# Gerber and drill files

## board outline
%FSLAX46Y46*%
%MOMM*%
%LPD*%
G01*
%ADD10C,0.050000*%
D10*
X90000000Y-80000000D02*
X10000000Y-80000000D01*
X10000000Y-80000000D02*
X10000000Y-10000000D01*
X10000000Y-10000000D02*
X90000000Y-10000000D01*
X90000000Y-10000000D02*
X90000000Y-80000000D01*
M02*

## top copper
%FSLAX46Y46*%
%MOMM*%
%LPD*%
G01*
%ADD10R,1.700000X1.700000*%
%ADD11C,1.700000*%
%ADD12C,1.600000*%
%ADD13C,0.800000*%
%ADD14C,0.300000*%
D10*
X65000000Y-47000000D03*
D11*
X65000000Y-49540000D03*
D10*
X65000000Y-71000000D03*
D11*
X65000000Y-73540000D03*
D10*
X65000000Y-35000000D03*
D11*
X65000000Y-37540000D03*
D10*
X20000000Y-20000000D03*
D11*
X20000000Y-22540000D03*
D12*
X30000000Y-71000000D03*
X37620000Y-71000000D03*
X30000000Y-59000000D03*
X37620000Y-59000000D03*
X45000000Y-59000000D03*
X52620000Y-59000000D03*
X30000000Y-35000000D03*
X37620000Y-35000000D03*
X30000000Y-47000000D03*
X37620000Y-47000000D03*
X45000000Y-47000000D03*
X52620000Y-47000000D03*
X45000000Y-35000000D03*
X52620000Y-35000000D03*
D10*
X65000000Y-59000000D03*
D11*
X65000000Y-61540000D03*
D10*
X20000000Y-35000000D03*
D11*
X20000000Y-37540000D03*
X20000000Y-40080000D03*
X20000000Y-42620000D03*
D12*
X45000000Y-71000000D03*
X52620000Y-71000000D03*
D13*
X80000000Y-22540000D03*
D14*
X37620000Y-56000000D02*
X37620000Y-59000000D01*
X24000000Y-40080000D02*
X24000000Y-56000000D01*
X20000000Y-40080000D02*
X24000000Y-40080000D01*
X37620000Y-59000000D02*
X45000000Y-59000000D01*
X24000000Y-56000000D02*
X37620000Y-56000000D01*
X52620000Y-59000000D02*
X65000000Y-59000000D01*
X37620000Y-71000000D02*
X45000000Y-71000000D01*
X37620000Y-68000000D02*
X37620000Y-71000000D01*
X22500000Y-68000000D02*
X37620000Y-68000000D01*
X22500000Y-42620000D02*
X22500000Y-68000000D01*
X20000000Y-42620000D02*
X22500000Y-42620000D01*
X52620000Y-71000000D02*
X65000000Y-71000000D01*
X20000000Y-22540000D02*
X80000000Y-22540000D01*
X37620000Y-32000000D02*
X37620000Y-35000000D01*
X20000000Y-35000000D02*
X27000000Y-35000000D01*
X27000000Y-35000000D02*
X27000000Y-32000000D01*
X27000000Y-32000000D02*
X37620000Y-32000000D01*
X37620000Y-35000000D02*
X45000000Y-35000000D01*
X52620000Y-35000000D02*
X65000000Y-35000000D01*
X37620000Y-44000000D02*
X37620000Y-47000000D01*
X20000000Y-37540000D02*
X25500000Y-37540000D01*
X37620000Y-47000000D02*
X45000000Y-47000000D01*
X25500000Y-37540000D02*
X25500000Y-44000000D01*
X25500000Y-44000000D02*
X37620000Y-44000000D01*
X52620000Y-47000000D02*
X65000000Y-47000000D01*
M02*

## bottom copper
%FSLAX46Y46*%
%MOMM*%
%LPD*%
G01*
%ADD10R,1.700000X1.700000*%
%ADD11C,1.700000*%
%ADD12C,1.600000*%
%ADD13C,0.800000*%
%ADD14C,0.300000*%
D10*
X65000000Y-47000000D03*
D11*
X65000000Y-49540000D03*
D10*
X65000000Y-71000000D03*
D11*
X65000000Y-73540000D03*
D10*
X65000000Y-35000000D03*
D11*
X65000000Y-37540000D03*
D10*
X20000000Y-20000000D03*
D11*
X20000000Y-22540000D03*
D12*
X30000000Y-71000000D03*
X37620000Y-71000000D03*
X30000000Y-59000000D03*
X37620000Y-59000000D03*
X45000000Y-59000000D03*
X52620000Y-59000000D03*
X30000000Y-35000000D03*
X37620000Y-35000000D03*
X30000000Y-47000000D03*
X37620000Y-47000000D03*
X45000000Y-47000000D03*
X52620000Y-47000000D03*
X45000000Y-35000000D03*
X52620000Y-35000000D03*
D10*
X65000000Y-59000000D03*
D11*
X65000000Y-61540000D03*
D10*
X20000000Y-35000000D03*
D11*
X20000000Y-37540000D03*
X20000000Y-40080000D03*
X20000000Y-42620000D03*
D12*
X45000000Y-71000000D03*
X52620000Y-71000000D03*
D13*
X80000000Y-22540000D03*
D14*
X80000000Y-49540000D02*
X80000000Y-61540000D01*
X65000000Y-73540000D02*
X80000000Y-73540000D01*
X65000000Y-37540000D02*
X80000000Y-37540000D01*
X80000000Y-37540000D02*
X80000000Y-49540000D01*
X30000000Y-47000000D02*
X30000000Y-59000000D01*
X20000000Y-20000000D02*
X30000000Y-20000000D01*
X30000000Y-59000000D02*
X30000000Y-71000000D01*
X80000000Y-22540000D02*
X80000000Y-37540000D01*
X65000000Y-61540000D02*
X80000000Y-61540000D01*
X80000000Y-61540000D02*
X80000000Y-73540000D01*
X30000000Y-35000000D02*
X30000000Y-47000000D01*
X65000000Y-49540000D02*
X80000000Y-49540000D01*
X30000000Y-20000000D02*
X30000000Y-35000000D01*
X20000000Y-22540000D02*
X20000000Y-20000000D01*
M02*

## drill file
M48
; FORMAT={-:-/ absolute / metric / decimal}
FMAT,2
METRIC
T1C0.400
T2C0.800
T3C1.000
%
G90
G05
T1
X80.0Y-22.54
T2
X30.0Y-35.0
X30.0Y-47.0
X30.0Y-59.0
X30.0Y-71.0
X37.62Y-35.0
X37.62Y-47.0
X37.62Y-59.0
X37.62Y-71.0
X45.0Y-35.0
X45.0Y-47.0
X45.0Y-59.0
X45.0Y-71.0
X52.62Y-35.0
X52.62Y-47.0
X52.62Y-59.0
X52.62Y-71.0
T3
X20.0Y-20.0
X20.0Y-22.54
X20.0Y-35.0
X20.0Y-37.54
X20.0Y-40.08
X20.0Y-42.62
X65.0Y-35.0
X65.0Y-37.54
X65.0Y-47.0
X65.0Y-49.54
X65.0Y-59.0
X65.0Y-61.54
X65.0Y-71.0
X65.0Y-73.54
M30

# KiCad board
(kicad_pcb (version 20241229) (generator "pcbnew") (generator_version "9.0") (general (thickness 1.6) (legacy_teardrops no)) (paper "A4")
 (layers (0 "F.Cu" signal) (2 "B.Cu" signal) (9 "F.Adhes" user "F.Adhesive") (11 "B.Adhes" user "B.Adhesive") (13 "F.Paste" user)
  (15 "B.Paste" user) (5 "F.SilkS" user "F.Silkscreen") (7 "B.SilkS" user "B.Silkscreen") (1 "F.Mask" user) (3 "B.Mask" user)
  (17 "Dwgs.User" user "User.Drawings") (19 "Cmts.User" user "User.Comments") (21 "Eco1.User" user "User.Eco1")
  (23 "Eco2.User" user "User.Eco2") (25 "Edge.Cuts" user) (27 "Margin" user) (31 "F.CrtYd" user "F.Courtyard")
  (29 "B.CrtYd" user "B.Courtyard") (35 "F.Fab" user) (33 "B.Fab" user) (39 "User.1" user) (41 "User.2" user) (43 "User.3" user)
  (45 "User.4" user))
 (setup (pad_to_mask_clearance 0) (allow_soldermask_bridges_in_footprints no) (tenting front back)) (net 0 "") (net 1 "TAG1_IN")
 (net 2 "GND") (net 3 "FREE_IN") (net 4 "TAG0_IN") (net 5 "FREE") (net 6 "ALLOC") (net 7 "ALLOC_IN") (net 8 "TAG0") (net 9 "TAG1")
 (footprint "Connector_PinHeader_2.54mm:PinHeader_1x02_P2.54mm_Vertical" (layer "F.Cu") (at 65 47)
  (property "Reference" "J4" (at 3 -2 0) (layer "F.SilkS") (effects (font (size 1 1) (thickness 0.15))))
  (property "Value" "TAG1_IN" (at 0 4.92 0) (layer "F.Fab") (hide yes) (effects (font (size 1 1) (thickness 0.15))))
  (pad "1" thru_hole rect (at 0 0) (size 1.7 1.7) (drill 1) (layers "*.Cu" "*.Mask") (remove_unused_layers no) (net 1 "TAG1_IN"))
  (pad "2" thru_hole circle (at 0 2.54) (size 1.7 1.7) (drill 1) (layers "*.Cu" "*.Mask") (remove_unused_layers no) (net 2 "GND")))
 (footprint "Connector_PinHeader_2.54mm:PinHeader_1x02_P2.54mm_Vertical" (layer "F.Cu") (at 65 71)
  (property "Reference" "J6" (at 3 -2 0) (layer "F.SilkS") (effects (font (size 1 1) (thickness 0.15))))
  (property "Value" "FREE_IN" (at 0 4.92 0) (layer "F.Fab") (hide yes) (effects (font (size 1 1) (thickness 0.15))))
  (pad "1" thru_hole rect (at 0 0) (size 1.7 1.7) (drill 1) (layers "*.Cu" "*.Mask") (remove_unused_layers no) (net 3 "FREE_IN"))
  (pad "2" thru_hole circle (at 0 2.54) (size 1.7 1.7) (drill 1) (layers "*.Cu" "*.Mask") (remove_unused_layers no) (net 2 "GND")))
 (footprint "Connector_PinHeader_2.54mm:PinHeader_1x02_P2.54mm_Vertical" (layer "F.Cu") (at 65 35)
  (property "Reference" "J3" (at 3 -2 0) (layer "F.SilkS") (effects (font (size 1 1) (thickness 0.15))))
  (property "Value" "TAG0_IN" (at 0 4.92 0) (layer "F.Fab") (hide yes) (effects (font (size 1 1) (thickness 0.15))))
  (pad "1" thru_hole rect (at 0 0) (size 1.7 1.7) (drill 1) (layers "*.Cu" "*.Mask") (remove_unused_layers no) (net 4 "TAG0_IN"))
  (pad "2" thru_hole circle (at 0 2.54) (size 1.7 1.7) (drill 1) (layers "*.Cu" "*.Mask") (remove_unused_layers no) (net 2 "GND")))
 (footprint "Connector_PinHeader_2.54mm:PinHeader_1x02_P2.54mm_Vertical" (layer "F.Cu") (at 20 20)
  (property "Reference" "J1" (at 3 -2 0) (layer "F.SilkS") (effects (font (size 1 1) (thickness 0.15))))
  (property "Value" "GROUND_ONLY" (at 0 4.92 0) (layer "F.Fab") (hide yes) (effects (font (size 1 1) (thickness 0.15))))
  (pad "1" thru_hole rect (at 0 0) (size 1.7 1.7) (drill 1) (layers "*.Cu" "*.Mask") (remove_unused_layers no) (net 2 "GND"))
  (pad "2" thru_hole circle (at 0 2.54) (size 1.7 1.7) (drill 1) (layers "*.Cu" "*.Mask") (remove_unused_layers no) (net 2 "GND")))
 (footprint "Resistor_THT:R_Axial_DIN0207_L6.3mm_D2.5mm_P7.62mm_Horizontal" (layer "F.Cu") (at 30 71)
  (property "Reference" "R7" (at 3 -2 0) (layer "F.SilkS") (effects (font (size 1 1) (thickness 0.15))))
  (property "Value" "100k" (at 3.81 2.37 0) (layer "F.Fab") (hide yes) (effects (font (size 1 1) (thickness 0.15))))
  (pad "1" thru_hole circle (at 0 0) (size 1.6 1.6) (drill 0.8) (layers "*.Cu" "*.Mask") (remove_unused_layers no) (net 2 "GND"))
  (pad "2" thru_hole circle (at 7.62 0) (size 1.6 1.6) (drill 0.8) (layers "*.Cu" "*.Mask") (remove_unused_layers no) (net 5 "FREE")))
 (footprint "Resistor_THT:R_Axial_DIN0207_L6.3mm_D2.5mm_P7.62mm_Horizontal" (layer "F.Cu") (at 30 59)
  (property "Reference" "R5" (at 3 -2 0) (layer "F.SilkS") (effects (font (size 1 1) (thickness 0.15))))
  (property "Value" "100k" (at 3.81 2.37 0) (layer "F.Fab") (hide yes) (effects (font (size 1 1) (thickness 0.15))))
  (pad "1" thru_hole circle (at 0 0) (size 1.6 1.6) (drill 0.8) (layers "*.Cu" "*.Mask") (remove_unused_layers no) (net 2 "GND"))
  (pad "2" thru_hole circle (at 7.62 0) (size 1.6 1.6) (drill 0.8) (layers "*.Cu" "*.Mask") (remove_unused_layers no) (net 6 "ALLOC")))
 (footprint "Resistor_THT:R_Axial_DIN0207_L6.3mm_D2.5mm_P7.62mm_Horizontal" (layer "F.Cu") (at 45 59)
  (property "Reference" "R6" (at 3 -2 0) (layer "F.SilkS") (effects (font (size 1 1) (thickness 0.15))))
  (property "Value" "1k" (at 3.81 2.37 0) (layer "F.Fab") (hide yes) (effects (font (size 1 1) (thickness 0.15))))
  (pad "1" thru_hole circle (at 0 0) (size 1.6 1.6) (drill 0.8) (layers "*.Cu" "*.Mask") (remove_unused_layers no) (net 6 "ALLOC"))
  (pad "2" thru_hole circle (at 7.62 0) (size 1.6 1.6) (drill 0.8) (layers "*.Cu" "*.Mask") (remove_unused_layers no) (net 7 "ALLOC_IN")))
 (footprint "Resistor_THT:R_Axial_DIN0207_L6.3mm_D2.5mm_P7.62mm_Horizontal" (layer "F.Cu") (at 30 35)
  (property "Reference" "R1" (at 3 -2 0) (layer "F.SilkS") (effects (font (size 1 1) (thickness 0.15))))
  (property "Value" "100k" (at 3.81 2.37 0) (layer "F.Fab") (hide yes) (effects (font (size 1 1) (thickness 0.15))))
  (pad "1" thru_hole circle (at 0 0) (size 1.6 1.6) (drill 0.8) (layers "*.Cu" "*.Mask") (remove_unused_layers no) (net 2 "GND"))
  (pad "2" thru_hole circle (at 7.62 0) (size 1.6 1.6) (drill 0.8) (layers "*.Cu" "*.Mask") (remove_unused_layers no) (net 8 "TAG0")))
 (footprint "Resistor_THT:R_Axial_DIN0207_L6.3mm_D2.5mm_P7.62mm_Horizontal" (layer "F.Cu") (at 30 47)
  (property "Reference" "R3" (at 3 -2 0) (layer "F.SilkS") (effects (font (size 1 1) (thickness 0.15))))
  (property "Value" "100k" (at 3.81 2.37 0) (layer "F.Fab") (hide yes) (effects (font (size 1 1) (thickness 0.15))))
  (pad "1" thru_hole circle (at 0 0) (size 1.6 1.6) (drill 0.8) (layers "*.Cu" "*.Mask") (remove_unused_layers no) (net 2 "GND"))
  (pad "2" thru_hole circle (at 7.62 0) (size 1.6 1.6) (drill 0.8) (layers "*.Cu" "*.Mask") (remove_unused_layers no) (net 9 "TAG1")))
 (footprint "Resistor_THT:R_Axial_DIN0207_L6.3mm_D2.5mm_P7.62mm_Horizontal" (layer "F.Cu") (at 45 47)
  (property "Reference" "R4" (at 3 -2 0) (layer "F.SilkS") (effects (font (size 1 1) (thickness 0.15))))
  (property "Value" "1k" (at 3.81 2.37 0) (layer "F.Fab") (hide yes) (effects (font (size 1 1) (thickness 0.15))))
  (pad "1" thru_hole circle (at 0 0) (size 1.6 1.6) (drill 0.8) (layers "*.Cu" "*.Mask") (remove_unused_layers no) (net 9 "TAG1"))
  (pad "2" thru_hole circle (at 7.62 0) (size 1.6 1.6) (drill 0.8) (layers "*.Cu" "*.Mask") (remove_unused_layers no) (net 1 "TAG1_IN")))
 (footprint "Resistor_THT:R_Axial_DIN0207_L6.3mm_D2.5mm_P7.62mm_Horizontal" (layer "F.Cu") (at 45 35)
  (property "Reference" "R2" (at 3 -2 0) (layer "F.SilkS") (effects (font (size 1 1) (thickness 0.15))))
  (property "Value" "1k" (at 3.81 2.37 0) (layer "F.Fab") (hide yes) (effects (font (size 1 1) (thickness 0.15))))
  (pad "1" thru_hole circle (at 0 0) (size 1.6 1.6) (drill 0.8) (layers "*.Cu" "*.Mask") (remove_unused_layers no) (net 8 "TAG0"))
  (pad "2" thru_hole circle (at 7.62 0) (size 1.6 1.6) (drill 0.8) (layers "*.Cu" "*.Mask") (remove_unused_layers no) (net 4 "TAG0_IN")))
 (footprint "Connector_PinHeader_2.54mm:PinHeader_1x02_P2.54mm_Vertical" (layer "F.Cu") (at 65 59)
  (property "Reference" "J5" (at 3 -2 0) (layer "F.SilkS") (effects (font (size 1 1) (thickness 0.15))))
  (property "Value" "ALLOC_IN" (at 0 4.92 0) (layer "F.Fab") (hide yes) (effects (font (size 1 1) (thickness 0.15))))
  (pad "1" thru_hole rect (at 0 0) (size 1.7 1.7) (drill 1) (layers "*.Cu" "*.Mask") (remove_unused_layers no) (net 7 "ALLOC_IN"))
  (pad "2" thru_hole circle (at 0 2.54) (size 1.7 1.7) (drill 1) (layers "*.Cu" "*.Mask") (remove_unused_layers no) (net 2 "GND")))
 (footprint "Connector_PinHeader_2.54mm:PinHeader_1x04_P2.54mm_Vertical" (layer "F.Cu") (at 20 35)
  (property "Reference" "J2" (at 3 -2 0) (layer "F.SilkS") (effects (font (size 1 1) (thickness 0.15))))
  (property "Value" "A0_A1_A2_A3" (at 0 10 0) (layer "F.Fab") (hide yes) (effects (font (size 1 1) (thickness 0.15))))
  (pad "1" thru_hole rect (at 0 0) (size 1.7 1.7) (drill 1) (layers "*.Cu" "*.Mask") (remove_unused_layers no) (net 8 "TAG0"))
  (pad "2" thru_hole circle (at 0 2.54) (size 1.7 1.7) (drill 1) (layers "*.Cu" "*.Mask") (remove_unused_layers no) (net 9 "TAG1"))
  (pad "3" thru_hole circle (at 0 5.08) (size 1.7 1.7) (drill 1) (layers "*.Cu" "*.Mask") (remove_unused_layers no) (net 6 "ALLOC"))
  (pad "4" thru_hole circle (at 0 7.62) (size 1.7 1.7) (drill 1) (layers "*.Cu" "*.Mask") (remove_unused_layers no) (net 5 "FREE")))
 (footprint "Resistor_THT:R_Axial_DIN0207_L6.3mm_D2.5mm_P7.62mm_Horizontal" (layer "F.Cu") (at 45 71)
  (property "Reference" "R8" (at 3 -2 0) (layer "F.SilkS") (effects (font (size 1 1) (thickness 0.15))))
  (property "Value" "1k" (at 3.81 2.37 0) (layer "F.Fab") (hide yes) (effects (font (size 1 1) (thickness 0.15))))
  (pad "1" thru_hole circle (at 0 0) (size 1.6 1.6) (drill 0.8) (layers "*.Cu" "*.Mask") (remove_unused_layers no) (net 5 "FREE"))
  (pad "2" thru_hole circle (at 7.62 0) (size 1.6 1.6) (drill 0.8) (layers "*.Cu" "*.Mask") (remove_unused_layers no) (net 3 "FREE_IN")))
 (gr_line (start 90 80) (end 10 80) (stroke (width 0.05) (type default)) (layer "Edge.Cuts"))
 (gr_line (start 10 80) (end 10 10) (stroke (width 0.05) (type default)) (layer "Edge.Cuts"))
 (gr_line (start 10 10) (end 90 10) (stroke (width 0.05) (type default)) (layer "Edge.Cuts"))
 (gr_line (start 90 10) (end 90 80) (stroke (width 0.05) (type default)) (layer "Edge.Cuts"))
 (segment (start 37.62 56) (end 37.62 59) (width 0.3) (layer "F.Cu") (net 6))
 (segment (start 24 40.08) (end 24 56) (width 0.3) (layer "F.Cu") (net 6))
 (segment (start 20 40.08) (end 24 40.08) (width 0.3) (layer "F.Cu") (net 6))
 (segment (start 37.62 59) (end 45 59) (width 0.3) (layer "F.Cu") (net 6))
 (segment (start 24 56) (end 37.62 56) (width 0.3) (layer "F.Cu") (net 6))
 (segment (start 52.62 59) (end 65 59) (width 0.3) (layer "F.Cu") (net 7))
 (segment (start 37.62 71) (end 45 71) (width 0.3) (layer "F.Cu") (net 5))
 (segment (start 37.62 68) (end 37.62 71) (width 0.3) (layer "F.Cu") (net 5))
 (segment (start 22.5 68) (end 37.62 68) (width 0.3) (layer "F.Cu") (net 5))
 (segment (start 22.5 42.62) (end 22.5 68) (width 0.3) (layer "F.Cu") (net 5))
 (segment (start 20 42.62) (end 22.5 42.62) (width 0.3) (layer "F.Cu") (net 5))
 (segment (start 52.62 71) (end 65 71) (width 0.3) (layer "F.Cu") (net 3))
 (segment (start 20 22.54) (end 80 22.54) (width 0.3) (layer "F.Cu") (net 2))
 (via (at 80 22.54) (size 0.8) (drill 0.4) (layers "F.Cu" "B.Cu") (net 2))
 (segment (start 80 49.54) (end 80 61.54) (width 0.3) (layer "B.Cu") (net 2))
 (segment (start 65 73.54) (end 80 73.54) (width 0.3) (layer "B.Cu") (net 2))
 (segment (start 65 37.54) (end 80 37.54) (width 0.3) (layer "B.Cu") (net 2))
 (segment (start 80 37.54) (end 80 49.54) (width 0.3) (layer "B.Cu") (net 2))
 (segment (start 30 47) (end 30 59) (width 0.3) (layer "B.Cu") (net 2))
 (segment (start 20 20) (end 30 20) (width 0.3) (layer "B.Cu") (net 2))
 (segment (start 30 59) (end 30 71) (width 0.3) (layer "B.Cu") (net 2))
 (segment (start 80 22.54) (end 80 37.54) (width 0.3) (layer "B.Cu") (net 2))
 (segment (start 65 61.54) (end 80 61.54) (width 0.3) (layer "B.Cu") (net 2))
 (segment (start 80 61.54) (end 80 73.54) (width 0.3) (layer "B.Cu") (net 2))
 (segment (start 30 35) (end 30 47) (width 0.3) (layer "B.Cu") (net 2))
 (segment (start 65 49.54) (end 80 49.54) (width 0.3) (layer "B.Cu") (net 2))
 (segment (start 30 20) (end 30 35) (width 0.3) (layer "B.Cu") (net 2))
 (segment (start 20 22.54) (end 20 20) (width 0.3) (layer "B.Cu") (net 2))
 (segment (start 37.62 32) (end 37.62 35) (width 0.3) (layer "F.Cu") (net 8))
 (segment (start 20 35) (end 27 35) (width 0.3) (layer "F.Cu") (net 8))
 (segment (start 27 35) (end 27 32) (width 0.3) (layer "F.Cu") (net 8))
 (segment (start 27 32) (end 37.62 32) (width 0.3) (layer "F.Cu") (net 8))
 (segment (start 37.62 35) (end 45 35) (width 0.3) (layer "F.Cu") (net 8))
 (segment (start 52.62 35) (end 65 35) (width 0.3) (layer "F.Cu") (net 4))
 (segment (start 37.62 44) (end 37.62 47) (width 0.3) (layer "F.Cu") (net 9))
 (segment (start 20 37.54) (end 25.5 37.54) (width 0.3) (layer "F.Cu") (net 9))
 (segment (start 37.62 47) (end 45 47) (width 0.3) (layer "F.Cu") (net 9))
 (segment (start 25.5 37.54) (end 25.5 44) (width 0.3) (layer "F.Cu") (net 9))
 (segment (start 25.5 44) (end 37.62 44) (width 0.3) (layer "F.Cu") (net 9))
 (segment (start 52.62 47) (end 65 47) (width 0.3) (layer "F.Cu") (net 1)))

